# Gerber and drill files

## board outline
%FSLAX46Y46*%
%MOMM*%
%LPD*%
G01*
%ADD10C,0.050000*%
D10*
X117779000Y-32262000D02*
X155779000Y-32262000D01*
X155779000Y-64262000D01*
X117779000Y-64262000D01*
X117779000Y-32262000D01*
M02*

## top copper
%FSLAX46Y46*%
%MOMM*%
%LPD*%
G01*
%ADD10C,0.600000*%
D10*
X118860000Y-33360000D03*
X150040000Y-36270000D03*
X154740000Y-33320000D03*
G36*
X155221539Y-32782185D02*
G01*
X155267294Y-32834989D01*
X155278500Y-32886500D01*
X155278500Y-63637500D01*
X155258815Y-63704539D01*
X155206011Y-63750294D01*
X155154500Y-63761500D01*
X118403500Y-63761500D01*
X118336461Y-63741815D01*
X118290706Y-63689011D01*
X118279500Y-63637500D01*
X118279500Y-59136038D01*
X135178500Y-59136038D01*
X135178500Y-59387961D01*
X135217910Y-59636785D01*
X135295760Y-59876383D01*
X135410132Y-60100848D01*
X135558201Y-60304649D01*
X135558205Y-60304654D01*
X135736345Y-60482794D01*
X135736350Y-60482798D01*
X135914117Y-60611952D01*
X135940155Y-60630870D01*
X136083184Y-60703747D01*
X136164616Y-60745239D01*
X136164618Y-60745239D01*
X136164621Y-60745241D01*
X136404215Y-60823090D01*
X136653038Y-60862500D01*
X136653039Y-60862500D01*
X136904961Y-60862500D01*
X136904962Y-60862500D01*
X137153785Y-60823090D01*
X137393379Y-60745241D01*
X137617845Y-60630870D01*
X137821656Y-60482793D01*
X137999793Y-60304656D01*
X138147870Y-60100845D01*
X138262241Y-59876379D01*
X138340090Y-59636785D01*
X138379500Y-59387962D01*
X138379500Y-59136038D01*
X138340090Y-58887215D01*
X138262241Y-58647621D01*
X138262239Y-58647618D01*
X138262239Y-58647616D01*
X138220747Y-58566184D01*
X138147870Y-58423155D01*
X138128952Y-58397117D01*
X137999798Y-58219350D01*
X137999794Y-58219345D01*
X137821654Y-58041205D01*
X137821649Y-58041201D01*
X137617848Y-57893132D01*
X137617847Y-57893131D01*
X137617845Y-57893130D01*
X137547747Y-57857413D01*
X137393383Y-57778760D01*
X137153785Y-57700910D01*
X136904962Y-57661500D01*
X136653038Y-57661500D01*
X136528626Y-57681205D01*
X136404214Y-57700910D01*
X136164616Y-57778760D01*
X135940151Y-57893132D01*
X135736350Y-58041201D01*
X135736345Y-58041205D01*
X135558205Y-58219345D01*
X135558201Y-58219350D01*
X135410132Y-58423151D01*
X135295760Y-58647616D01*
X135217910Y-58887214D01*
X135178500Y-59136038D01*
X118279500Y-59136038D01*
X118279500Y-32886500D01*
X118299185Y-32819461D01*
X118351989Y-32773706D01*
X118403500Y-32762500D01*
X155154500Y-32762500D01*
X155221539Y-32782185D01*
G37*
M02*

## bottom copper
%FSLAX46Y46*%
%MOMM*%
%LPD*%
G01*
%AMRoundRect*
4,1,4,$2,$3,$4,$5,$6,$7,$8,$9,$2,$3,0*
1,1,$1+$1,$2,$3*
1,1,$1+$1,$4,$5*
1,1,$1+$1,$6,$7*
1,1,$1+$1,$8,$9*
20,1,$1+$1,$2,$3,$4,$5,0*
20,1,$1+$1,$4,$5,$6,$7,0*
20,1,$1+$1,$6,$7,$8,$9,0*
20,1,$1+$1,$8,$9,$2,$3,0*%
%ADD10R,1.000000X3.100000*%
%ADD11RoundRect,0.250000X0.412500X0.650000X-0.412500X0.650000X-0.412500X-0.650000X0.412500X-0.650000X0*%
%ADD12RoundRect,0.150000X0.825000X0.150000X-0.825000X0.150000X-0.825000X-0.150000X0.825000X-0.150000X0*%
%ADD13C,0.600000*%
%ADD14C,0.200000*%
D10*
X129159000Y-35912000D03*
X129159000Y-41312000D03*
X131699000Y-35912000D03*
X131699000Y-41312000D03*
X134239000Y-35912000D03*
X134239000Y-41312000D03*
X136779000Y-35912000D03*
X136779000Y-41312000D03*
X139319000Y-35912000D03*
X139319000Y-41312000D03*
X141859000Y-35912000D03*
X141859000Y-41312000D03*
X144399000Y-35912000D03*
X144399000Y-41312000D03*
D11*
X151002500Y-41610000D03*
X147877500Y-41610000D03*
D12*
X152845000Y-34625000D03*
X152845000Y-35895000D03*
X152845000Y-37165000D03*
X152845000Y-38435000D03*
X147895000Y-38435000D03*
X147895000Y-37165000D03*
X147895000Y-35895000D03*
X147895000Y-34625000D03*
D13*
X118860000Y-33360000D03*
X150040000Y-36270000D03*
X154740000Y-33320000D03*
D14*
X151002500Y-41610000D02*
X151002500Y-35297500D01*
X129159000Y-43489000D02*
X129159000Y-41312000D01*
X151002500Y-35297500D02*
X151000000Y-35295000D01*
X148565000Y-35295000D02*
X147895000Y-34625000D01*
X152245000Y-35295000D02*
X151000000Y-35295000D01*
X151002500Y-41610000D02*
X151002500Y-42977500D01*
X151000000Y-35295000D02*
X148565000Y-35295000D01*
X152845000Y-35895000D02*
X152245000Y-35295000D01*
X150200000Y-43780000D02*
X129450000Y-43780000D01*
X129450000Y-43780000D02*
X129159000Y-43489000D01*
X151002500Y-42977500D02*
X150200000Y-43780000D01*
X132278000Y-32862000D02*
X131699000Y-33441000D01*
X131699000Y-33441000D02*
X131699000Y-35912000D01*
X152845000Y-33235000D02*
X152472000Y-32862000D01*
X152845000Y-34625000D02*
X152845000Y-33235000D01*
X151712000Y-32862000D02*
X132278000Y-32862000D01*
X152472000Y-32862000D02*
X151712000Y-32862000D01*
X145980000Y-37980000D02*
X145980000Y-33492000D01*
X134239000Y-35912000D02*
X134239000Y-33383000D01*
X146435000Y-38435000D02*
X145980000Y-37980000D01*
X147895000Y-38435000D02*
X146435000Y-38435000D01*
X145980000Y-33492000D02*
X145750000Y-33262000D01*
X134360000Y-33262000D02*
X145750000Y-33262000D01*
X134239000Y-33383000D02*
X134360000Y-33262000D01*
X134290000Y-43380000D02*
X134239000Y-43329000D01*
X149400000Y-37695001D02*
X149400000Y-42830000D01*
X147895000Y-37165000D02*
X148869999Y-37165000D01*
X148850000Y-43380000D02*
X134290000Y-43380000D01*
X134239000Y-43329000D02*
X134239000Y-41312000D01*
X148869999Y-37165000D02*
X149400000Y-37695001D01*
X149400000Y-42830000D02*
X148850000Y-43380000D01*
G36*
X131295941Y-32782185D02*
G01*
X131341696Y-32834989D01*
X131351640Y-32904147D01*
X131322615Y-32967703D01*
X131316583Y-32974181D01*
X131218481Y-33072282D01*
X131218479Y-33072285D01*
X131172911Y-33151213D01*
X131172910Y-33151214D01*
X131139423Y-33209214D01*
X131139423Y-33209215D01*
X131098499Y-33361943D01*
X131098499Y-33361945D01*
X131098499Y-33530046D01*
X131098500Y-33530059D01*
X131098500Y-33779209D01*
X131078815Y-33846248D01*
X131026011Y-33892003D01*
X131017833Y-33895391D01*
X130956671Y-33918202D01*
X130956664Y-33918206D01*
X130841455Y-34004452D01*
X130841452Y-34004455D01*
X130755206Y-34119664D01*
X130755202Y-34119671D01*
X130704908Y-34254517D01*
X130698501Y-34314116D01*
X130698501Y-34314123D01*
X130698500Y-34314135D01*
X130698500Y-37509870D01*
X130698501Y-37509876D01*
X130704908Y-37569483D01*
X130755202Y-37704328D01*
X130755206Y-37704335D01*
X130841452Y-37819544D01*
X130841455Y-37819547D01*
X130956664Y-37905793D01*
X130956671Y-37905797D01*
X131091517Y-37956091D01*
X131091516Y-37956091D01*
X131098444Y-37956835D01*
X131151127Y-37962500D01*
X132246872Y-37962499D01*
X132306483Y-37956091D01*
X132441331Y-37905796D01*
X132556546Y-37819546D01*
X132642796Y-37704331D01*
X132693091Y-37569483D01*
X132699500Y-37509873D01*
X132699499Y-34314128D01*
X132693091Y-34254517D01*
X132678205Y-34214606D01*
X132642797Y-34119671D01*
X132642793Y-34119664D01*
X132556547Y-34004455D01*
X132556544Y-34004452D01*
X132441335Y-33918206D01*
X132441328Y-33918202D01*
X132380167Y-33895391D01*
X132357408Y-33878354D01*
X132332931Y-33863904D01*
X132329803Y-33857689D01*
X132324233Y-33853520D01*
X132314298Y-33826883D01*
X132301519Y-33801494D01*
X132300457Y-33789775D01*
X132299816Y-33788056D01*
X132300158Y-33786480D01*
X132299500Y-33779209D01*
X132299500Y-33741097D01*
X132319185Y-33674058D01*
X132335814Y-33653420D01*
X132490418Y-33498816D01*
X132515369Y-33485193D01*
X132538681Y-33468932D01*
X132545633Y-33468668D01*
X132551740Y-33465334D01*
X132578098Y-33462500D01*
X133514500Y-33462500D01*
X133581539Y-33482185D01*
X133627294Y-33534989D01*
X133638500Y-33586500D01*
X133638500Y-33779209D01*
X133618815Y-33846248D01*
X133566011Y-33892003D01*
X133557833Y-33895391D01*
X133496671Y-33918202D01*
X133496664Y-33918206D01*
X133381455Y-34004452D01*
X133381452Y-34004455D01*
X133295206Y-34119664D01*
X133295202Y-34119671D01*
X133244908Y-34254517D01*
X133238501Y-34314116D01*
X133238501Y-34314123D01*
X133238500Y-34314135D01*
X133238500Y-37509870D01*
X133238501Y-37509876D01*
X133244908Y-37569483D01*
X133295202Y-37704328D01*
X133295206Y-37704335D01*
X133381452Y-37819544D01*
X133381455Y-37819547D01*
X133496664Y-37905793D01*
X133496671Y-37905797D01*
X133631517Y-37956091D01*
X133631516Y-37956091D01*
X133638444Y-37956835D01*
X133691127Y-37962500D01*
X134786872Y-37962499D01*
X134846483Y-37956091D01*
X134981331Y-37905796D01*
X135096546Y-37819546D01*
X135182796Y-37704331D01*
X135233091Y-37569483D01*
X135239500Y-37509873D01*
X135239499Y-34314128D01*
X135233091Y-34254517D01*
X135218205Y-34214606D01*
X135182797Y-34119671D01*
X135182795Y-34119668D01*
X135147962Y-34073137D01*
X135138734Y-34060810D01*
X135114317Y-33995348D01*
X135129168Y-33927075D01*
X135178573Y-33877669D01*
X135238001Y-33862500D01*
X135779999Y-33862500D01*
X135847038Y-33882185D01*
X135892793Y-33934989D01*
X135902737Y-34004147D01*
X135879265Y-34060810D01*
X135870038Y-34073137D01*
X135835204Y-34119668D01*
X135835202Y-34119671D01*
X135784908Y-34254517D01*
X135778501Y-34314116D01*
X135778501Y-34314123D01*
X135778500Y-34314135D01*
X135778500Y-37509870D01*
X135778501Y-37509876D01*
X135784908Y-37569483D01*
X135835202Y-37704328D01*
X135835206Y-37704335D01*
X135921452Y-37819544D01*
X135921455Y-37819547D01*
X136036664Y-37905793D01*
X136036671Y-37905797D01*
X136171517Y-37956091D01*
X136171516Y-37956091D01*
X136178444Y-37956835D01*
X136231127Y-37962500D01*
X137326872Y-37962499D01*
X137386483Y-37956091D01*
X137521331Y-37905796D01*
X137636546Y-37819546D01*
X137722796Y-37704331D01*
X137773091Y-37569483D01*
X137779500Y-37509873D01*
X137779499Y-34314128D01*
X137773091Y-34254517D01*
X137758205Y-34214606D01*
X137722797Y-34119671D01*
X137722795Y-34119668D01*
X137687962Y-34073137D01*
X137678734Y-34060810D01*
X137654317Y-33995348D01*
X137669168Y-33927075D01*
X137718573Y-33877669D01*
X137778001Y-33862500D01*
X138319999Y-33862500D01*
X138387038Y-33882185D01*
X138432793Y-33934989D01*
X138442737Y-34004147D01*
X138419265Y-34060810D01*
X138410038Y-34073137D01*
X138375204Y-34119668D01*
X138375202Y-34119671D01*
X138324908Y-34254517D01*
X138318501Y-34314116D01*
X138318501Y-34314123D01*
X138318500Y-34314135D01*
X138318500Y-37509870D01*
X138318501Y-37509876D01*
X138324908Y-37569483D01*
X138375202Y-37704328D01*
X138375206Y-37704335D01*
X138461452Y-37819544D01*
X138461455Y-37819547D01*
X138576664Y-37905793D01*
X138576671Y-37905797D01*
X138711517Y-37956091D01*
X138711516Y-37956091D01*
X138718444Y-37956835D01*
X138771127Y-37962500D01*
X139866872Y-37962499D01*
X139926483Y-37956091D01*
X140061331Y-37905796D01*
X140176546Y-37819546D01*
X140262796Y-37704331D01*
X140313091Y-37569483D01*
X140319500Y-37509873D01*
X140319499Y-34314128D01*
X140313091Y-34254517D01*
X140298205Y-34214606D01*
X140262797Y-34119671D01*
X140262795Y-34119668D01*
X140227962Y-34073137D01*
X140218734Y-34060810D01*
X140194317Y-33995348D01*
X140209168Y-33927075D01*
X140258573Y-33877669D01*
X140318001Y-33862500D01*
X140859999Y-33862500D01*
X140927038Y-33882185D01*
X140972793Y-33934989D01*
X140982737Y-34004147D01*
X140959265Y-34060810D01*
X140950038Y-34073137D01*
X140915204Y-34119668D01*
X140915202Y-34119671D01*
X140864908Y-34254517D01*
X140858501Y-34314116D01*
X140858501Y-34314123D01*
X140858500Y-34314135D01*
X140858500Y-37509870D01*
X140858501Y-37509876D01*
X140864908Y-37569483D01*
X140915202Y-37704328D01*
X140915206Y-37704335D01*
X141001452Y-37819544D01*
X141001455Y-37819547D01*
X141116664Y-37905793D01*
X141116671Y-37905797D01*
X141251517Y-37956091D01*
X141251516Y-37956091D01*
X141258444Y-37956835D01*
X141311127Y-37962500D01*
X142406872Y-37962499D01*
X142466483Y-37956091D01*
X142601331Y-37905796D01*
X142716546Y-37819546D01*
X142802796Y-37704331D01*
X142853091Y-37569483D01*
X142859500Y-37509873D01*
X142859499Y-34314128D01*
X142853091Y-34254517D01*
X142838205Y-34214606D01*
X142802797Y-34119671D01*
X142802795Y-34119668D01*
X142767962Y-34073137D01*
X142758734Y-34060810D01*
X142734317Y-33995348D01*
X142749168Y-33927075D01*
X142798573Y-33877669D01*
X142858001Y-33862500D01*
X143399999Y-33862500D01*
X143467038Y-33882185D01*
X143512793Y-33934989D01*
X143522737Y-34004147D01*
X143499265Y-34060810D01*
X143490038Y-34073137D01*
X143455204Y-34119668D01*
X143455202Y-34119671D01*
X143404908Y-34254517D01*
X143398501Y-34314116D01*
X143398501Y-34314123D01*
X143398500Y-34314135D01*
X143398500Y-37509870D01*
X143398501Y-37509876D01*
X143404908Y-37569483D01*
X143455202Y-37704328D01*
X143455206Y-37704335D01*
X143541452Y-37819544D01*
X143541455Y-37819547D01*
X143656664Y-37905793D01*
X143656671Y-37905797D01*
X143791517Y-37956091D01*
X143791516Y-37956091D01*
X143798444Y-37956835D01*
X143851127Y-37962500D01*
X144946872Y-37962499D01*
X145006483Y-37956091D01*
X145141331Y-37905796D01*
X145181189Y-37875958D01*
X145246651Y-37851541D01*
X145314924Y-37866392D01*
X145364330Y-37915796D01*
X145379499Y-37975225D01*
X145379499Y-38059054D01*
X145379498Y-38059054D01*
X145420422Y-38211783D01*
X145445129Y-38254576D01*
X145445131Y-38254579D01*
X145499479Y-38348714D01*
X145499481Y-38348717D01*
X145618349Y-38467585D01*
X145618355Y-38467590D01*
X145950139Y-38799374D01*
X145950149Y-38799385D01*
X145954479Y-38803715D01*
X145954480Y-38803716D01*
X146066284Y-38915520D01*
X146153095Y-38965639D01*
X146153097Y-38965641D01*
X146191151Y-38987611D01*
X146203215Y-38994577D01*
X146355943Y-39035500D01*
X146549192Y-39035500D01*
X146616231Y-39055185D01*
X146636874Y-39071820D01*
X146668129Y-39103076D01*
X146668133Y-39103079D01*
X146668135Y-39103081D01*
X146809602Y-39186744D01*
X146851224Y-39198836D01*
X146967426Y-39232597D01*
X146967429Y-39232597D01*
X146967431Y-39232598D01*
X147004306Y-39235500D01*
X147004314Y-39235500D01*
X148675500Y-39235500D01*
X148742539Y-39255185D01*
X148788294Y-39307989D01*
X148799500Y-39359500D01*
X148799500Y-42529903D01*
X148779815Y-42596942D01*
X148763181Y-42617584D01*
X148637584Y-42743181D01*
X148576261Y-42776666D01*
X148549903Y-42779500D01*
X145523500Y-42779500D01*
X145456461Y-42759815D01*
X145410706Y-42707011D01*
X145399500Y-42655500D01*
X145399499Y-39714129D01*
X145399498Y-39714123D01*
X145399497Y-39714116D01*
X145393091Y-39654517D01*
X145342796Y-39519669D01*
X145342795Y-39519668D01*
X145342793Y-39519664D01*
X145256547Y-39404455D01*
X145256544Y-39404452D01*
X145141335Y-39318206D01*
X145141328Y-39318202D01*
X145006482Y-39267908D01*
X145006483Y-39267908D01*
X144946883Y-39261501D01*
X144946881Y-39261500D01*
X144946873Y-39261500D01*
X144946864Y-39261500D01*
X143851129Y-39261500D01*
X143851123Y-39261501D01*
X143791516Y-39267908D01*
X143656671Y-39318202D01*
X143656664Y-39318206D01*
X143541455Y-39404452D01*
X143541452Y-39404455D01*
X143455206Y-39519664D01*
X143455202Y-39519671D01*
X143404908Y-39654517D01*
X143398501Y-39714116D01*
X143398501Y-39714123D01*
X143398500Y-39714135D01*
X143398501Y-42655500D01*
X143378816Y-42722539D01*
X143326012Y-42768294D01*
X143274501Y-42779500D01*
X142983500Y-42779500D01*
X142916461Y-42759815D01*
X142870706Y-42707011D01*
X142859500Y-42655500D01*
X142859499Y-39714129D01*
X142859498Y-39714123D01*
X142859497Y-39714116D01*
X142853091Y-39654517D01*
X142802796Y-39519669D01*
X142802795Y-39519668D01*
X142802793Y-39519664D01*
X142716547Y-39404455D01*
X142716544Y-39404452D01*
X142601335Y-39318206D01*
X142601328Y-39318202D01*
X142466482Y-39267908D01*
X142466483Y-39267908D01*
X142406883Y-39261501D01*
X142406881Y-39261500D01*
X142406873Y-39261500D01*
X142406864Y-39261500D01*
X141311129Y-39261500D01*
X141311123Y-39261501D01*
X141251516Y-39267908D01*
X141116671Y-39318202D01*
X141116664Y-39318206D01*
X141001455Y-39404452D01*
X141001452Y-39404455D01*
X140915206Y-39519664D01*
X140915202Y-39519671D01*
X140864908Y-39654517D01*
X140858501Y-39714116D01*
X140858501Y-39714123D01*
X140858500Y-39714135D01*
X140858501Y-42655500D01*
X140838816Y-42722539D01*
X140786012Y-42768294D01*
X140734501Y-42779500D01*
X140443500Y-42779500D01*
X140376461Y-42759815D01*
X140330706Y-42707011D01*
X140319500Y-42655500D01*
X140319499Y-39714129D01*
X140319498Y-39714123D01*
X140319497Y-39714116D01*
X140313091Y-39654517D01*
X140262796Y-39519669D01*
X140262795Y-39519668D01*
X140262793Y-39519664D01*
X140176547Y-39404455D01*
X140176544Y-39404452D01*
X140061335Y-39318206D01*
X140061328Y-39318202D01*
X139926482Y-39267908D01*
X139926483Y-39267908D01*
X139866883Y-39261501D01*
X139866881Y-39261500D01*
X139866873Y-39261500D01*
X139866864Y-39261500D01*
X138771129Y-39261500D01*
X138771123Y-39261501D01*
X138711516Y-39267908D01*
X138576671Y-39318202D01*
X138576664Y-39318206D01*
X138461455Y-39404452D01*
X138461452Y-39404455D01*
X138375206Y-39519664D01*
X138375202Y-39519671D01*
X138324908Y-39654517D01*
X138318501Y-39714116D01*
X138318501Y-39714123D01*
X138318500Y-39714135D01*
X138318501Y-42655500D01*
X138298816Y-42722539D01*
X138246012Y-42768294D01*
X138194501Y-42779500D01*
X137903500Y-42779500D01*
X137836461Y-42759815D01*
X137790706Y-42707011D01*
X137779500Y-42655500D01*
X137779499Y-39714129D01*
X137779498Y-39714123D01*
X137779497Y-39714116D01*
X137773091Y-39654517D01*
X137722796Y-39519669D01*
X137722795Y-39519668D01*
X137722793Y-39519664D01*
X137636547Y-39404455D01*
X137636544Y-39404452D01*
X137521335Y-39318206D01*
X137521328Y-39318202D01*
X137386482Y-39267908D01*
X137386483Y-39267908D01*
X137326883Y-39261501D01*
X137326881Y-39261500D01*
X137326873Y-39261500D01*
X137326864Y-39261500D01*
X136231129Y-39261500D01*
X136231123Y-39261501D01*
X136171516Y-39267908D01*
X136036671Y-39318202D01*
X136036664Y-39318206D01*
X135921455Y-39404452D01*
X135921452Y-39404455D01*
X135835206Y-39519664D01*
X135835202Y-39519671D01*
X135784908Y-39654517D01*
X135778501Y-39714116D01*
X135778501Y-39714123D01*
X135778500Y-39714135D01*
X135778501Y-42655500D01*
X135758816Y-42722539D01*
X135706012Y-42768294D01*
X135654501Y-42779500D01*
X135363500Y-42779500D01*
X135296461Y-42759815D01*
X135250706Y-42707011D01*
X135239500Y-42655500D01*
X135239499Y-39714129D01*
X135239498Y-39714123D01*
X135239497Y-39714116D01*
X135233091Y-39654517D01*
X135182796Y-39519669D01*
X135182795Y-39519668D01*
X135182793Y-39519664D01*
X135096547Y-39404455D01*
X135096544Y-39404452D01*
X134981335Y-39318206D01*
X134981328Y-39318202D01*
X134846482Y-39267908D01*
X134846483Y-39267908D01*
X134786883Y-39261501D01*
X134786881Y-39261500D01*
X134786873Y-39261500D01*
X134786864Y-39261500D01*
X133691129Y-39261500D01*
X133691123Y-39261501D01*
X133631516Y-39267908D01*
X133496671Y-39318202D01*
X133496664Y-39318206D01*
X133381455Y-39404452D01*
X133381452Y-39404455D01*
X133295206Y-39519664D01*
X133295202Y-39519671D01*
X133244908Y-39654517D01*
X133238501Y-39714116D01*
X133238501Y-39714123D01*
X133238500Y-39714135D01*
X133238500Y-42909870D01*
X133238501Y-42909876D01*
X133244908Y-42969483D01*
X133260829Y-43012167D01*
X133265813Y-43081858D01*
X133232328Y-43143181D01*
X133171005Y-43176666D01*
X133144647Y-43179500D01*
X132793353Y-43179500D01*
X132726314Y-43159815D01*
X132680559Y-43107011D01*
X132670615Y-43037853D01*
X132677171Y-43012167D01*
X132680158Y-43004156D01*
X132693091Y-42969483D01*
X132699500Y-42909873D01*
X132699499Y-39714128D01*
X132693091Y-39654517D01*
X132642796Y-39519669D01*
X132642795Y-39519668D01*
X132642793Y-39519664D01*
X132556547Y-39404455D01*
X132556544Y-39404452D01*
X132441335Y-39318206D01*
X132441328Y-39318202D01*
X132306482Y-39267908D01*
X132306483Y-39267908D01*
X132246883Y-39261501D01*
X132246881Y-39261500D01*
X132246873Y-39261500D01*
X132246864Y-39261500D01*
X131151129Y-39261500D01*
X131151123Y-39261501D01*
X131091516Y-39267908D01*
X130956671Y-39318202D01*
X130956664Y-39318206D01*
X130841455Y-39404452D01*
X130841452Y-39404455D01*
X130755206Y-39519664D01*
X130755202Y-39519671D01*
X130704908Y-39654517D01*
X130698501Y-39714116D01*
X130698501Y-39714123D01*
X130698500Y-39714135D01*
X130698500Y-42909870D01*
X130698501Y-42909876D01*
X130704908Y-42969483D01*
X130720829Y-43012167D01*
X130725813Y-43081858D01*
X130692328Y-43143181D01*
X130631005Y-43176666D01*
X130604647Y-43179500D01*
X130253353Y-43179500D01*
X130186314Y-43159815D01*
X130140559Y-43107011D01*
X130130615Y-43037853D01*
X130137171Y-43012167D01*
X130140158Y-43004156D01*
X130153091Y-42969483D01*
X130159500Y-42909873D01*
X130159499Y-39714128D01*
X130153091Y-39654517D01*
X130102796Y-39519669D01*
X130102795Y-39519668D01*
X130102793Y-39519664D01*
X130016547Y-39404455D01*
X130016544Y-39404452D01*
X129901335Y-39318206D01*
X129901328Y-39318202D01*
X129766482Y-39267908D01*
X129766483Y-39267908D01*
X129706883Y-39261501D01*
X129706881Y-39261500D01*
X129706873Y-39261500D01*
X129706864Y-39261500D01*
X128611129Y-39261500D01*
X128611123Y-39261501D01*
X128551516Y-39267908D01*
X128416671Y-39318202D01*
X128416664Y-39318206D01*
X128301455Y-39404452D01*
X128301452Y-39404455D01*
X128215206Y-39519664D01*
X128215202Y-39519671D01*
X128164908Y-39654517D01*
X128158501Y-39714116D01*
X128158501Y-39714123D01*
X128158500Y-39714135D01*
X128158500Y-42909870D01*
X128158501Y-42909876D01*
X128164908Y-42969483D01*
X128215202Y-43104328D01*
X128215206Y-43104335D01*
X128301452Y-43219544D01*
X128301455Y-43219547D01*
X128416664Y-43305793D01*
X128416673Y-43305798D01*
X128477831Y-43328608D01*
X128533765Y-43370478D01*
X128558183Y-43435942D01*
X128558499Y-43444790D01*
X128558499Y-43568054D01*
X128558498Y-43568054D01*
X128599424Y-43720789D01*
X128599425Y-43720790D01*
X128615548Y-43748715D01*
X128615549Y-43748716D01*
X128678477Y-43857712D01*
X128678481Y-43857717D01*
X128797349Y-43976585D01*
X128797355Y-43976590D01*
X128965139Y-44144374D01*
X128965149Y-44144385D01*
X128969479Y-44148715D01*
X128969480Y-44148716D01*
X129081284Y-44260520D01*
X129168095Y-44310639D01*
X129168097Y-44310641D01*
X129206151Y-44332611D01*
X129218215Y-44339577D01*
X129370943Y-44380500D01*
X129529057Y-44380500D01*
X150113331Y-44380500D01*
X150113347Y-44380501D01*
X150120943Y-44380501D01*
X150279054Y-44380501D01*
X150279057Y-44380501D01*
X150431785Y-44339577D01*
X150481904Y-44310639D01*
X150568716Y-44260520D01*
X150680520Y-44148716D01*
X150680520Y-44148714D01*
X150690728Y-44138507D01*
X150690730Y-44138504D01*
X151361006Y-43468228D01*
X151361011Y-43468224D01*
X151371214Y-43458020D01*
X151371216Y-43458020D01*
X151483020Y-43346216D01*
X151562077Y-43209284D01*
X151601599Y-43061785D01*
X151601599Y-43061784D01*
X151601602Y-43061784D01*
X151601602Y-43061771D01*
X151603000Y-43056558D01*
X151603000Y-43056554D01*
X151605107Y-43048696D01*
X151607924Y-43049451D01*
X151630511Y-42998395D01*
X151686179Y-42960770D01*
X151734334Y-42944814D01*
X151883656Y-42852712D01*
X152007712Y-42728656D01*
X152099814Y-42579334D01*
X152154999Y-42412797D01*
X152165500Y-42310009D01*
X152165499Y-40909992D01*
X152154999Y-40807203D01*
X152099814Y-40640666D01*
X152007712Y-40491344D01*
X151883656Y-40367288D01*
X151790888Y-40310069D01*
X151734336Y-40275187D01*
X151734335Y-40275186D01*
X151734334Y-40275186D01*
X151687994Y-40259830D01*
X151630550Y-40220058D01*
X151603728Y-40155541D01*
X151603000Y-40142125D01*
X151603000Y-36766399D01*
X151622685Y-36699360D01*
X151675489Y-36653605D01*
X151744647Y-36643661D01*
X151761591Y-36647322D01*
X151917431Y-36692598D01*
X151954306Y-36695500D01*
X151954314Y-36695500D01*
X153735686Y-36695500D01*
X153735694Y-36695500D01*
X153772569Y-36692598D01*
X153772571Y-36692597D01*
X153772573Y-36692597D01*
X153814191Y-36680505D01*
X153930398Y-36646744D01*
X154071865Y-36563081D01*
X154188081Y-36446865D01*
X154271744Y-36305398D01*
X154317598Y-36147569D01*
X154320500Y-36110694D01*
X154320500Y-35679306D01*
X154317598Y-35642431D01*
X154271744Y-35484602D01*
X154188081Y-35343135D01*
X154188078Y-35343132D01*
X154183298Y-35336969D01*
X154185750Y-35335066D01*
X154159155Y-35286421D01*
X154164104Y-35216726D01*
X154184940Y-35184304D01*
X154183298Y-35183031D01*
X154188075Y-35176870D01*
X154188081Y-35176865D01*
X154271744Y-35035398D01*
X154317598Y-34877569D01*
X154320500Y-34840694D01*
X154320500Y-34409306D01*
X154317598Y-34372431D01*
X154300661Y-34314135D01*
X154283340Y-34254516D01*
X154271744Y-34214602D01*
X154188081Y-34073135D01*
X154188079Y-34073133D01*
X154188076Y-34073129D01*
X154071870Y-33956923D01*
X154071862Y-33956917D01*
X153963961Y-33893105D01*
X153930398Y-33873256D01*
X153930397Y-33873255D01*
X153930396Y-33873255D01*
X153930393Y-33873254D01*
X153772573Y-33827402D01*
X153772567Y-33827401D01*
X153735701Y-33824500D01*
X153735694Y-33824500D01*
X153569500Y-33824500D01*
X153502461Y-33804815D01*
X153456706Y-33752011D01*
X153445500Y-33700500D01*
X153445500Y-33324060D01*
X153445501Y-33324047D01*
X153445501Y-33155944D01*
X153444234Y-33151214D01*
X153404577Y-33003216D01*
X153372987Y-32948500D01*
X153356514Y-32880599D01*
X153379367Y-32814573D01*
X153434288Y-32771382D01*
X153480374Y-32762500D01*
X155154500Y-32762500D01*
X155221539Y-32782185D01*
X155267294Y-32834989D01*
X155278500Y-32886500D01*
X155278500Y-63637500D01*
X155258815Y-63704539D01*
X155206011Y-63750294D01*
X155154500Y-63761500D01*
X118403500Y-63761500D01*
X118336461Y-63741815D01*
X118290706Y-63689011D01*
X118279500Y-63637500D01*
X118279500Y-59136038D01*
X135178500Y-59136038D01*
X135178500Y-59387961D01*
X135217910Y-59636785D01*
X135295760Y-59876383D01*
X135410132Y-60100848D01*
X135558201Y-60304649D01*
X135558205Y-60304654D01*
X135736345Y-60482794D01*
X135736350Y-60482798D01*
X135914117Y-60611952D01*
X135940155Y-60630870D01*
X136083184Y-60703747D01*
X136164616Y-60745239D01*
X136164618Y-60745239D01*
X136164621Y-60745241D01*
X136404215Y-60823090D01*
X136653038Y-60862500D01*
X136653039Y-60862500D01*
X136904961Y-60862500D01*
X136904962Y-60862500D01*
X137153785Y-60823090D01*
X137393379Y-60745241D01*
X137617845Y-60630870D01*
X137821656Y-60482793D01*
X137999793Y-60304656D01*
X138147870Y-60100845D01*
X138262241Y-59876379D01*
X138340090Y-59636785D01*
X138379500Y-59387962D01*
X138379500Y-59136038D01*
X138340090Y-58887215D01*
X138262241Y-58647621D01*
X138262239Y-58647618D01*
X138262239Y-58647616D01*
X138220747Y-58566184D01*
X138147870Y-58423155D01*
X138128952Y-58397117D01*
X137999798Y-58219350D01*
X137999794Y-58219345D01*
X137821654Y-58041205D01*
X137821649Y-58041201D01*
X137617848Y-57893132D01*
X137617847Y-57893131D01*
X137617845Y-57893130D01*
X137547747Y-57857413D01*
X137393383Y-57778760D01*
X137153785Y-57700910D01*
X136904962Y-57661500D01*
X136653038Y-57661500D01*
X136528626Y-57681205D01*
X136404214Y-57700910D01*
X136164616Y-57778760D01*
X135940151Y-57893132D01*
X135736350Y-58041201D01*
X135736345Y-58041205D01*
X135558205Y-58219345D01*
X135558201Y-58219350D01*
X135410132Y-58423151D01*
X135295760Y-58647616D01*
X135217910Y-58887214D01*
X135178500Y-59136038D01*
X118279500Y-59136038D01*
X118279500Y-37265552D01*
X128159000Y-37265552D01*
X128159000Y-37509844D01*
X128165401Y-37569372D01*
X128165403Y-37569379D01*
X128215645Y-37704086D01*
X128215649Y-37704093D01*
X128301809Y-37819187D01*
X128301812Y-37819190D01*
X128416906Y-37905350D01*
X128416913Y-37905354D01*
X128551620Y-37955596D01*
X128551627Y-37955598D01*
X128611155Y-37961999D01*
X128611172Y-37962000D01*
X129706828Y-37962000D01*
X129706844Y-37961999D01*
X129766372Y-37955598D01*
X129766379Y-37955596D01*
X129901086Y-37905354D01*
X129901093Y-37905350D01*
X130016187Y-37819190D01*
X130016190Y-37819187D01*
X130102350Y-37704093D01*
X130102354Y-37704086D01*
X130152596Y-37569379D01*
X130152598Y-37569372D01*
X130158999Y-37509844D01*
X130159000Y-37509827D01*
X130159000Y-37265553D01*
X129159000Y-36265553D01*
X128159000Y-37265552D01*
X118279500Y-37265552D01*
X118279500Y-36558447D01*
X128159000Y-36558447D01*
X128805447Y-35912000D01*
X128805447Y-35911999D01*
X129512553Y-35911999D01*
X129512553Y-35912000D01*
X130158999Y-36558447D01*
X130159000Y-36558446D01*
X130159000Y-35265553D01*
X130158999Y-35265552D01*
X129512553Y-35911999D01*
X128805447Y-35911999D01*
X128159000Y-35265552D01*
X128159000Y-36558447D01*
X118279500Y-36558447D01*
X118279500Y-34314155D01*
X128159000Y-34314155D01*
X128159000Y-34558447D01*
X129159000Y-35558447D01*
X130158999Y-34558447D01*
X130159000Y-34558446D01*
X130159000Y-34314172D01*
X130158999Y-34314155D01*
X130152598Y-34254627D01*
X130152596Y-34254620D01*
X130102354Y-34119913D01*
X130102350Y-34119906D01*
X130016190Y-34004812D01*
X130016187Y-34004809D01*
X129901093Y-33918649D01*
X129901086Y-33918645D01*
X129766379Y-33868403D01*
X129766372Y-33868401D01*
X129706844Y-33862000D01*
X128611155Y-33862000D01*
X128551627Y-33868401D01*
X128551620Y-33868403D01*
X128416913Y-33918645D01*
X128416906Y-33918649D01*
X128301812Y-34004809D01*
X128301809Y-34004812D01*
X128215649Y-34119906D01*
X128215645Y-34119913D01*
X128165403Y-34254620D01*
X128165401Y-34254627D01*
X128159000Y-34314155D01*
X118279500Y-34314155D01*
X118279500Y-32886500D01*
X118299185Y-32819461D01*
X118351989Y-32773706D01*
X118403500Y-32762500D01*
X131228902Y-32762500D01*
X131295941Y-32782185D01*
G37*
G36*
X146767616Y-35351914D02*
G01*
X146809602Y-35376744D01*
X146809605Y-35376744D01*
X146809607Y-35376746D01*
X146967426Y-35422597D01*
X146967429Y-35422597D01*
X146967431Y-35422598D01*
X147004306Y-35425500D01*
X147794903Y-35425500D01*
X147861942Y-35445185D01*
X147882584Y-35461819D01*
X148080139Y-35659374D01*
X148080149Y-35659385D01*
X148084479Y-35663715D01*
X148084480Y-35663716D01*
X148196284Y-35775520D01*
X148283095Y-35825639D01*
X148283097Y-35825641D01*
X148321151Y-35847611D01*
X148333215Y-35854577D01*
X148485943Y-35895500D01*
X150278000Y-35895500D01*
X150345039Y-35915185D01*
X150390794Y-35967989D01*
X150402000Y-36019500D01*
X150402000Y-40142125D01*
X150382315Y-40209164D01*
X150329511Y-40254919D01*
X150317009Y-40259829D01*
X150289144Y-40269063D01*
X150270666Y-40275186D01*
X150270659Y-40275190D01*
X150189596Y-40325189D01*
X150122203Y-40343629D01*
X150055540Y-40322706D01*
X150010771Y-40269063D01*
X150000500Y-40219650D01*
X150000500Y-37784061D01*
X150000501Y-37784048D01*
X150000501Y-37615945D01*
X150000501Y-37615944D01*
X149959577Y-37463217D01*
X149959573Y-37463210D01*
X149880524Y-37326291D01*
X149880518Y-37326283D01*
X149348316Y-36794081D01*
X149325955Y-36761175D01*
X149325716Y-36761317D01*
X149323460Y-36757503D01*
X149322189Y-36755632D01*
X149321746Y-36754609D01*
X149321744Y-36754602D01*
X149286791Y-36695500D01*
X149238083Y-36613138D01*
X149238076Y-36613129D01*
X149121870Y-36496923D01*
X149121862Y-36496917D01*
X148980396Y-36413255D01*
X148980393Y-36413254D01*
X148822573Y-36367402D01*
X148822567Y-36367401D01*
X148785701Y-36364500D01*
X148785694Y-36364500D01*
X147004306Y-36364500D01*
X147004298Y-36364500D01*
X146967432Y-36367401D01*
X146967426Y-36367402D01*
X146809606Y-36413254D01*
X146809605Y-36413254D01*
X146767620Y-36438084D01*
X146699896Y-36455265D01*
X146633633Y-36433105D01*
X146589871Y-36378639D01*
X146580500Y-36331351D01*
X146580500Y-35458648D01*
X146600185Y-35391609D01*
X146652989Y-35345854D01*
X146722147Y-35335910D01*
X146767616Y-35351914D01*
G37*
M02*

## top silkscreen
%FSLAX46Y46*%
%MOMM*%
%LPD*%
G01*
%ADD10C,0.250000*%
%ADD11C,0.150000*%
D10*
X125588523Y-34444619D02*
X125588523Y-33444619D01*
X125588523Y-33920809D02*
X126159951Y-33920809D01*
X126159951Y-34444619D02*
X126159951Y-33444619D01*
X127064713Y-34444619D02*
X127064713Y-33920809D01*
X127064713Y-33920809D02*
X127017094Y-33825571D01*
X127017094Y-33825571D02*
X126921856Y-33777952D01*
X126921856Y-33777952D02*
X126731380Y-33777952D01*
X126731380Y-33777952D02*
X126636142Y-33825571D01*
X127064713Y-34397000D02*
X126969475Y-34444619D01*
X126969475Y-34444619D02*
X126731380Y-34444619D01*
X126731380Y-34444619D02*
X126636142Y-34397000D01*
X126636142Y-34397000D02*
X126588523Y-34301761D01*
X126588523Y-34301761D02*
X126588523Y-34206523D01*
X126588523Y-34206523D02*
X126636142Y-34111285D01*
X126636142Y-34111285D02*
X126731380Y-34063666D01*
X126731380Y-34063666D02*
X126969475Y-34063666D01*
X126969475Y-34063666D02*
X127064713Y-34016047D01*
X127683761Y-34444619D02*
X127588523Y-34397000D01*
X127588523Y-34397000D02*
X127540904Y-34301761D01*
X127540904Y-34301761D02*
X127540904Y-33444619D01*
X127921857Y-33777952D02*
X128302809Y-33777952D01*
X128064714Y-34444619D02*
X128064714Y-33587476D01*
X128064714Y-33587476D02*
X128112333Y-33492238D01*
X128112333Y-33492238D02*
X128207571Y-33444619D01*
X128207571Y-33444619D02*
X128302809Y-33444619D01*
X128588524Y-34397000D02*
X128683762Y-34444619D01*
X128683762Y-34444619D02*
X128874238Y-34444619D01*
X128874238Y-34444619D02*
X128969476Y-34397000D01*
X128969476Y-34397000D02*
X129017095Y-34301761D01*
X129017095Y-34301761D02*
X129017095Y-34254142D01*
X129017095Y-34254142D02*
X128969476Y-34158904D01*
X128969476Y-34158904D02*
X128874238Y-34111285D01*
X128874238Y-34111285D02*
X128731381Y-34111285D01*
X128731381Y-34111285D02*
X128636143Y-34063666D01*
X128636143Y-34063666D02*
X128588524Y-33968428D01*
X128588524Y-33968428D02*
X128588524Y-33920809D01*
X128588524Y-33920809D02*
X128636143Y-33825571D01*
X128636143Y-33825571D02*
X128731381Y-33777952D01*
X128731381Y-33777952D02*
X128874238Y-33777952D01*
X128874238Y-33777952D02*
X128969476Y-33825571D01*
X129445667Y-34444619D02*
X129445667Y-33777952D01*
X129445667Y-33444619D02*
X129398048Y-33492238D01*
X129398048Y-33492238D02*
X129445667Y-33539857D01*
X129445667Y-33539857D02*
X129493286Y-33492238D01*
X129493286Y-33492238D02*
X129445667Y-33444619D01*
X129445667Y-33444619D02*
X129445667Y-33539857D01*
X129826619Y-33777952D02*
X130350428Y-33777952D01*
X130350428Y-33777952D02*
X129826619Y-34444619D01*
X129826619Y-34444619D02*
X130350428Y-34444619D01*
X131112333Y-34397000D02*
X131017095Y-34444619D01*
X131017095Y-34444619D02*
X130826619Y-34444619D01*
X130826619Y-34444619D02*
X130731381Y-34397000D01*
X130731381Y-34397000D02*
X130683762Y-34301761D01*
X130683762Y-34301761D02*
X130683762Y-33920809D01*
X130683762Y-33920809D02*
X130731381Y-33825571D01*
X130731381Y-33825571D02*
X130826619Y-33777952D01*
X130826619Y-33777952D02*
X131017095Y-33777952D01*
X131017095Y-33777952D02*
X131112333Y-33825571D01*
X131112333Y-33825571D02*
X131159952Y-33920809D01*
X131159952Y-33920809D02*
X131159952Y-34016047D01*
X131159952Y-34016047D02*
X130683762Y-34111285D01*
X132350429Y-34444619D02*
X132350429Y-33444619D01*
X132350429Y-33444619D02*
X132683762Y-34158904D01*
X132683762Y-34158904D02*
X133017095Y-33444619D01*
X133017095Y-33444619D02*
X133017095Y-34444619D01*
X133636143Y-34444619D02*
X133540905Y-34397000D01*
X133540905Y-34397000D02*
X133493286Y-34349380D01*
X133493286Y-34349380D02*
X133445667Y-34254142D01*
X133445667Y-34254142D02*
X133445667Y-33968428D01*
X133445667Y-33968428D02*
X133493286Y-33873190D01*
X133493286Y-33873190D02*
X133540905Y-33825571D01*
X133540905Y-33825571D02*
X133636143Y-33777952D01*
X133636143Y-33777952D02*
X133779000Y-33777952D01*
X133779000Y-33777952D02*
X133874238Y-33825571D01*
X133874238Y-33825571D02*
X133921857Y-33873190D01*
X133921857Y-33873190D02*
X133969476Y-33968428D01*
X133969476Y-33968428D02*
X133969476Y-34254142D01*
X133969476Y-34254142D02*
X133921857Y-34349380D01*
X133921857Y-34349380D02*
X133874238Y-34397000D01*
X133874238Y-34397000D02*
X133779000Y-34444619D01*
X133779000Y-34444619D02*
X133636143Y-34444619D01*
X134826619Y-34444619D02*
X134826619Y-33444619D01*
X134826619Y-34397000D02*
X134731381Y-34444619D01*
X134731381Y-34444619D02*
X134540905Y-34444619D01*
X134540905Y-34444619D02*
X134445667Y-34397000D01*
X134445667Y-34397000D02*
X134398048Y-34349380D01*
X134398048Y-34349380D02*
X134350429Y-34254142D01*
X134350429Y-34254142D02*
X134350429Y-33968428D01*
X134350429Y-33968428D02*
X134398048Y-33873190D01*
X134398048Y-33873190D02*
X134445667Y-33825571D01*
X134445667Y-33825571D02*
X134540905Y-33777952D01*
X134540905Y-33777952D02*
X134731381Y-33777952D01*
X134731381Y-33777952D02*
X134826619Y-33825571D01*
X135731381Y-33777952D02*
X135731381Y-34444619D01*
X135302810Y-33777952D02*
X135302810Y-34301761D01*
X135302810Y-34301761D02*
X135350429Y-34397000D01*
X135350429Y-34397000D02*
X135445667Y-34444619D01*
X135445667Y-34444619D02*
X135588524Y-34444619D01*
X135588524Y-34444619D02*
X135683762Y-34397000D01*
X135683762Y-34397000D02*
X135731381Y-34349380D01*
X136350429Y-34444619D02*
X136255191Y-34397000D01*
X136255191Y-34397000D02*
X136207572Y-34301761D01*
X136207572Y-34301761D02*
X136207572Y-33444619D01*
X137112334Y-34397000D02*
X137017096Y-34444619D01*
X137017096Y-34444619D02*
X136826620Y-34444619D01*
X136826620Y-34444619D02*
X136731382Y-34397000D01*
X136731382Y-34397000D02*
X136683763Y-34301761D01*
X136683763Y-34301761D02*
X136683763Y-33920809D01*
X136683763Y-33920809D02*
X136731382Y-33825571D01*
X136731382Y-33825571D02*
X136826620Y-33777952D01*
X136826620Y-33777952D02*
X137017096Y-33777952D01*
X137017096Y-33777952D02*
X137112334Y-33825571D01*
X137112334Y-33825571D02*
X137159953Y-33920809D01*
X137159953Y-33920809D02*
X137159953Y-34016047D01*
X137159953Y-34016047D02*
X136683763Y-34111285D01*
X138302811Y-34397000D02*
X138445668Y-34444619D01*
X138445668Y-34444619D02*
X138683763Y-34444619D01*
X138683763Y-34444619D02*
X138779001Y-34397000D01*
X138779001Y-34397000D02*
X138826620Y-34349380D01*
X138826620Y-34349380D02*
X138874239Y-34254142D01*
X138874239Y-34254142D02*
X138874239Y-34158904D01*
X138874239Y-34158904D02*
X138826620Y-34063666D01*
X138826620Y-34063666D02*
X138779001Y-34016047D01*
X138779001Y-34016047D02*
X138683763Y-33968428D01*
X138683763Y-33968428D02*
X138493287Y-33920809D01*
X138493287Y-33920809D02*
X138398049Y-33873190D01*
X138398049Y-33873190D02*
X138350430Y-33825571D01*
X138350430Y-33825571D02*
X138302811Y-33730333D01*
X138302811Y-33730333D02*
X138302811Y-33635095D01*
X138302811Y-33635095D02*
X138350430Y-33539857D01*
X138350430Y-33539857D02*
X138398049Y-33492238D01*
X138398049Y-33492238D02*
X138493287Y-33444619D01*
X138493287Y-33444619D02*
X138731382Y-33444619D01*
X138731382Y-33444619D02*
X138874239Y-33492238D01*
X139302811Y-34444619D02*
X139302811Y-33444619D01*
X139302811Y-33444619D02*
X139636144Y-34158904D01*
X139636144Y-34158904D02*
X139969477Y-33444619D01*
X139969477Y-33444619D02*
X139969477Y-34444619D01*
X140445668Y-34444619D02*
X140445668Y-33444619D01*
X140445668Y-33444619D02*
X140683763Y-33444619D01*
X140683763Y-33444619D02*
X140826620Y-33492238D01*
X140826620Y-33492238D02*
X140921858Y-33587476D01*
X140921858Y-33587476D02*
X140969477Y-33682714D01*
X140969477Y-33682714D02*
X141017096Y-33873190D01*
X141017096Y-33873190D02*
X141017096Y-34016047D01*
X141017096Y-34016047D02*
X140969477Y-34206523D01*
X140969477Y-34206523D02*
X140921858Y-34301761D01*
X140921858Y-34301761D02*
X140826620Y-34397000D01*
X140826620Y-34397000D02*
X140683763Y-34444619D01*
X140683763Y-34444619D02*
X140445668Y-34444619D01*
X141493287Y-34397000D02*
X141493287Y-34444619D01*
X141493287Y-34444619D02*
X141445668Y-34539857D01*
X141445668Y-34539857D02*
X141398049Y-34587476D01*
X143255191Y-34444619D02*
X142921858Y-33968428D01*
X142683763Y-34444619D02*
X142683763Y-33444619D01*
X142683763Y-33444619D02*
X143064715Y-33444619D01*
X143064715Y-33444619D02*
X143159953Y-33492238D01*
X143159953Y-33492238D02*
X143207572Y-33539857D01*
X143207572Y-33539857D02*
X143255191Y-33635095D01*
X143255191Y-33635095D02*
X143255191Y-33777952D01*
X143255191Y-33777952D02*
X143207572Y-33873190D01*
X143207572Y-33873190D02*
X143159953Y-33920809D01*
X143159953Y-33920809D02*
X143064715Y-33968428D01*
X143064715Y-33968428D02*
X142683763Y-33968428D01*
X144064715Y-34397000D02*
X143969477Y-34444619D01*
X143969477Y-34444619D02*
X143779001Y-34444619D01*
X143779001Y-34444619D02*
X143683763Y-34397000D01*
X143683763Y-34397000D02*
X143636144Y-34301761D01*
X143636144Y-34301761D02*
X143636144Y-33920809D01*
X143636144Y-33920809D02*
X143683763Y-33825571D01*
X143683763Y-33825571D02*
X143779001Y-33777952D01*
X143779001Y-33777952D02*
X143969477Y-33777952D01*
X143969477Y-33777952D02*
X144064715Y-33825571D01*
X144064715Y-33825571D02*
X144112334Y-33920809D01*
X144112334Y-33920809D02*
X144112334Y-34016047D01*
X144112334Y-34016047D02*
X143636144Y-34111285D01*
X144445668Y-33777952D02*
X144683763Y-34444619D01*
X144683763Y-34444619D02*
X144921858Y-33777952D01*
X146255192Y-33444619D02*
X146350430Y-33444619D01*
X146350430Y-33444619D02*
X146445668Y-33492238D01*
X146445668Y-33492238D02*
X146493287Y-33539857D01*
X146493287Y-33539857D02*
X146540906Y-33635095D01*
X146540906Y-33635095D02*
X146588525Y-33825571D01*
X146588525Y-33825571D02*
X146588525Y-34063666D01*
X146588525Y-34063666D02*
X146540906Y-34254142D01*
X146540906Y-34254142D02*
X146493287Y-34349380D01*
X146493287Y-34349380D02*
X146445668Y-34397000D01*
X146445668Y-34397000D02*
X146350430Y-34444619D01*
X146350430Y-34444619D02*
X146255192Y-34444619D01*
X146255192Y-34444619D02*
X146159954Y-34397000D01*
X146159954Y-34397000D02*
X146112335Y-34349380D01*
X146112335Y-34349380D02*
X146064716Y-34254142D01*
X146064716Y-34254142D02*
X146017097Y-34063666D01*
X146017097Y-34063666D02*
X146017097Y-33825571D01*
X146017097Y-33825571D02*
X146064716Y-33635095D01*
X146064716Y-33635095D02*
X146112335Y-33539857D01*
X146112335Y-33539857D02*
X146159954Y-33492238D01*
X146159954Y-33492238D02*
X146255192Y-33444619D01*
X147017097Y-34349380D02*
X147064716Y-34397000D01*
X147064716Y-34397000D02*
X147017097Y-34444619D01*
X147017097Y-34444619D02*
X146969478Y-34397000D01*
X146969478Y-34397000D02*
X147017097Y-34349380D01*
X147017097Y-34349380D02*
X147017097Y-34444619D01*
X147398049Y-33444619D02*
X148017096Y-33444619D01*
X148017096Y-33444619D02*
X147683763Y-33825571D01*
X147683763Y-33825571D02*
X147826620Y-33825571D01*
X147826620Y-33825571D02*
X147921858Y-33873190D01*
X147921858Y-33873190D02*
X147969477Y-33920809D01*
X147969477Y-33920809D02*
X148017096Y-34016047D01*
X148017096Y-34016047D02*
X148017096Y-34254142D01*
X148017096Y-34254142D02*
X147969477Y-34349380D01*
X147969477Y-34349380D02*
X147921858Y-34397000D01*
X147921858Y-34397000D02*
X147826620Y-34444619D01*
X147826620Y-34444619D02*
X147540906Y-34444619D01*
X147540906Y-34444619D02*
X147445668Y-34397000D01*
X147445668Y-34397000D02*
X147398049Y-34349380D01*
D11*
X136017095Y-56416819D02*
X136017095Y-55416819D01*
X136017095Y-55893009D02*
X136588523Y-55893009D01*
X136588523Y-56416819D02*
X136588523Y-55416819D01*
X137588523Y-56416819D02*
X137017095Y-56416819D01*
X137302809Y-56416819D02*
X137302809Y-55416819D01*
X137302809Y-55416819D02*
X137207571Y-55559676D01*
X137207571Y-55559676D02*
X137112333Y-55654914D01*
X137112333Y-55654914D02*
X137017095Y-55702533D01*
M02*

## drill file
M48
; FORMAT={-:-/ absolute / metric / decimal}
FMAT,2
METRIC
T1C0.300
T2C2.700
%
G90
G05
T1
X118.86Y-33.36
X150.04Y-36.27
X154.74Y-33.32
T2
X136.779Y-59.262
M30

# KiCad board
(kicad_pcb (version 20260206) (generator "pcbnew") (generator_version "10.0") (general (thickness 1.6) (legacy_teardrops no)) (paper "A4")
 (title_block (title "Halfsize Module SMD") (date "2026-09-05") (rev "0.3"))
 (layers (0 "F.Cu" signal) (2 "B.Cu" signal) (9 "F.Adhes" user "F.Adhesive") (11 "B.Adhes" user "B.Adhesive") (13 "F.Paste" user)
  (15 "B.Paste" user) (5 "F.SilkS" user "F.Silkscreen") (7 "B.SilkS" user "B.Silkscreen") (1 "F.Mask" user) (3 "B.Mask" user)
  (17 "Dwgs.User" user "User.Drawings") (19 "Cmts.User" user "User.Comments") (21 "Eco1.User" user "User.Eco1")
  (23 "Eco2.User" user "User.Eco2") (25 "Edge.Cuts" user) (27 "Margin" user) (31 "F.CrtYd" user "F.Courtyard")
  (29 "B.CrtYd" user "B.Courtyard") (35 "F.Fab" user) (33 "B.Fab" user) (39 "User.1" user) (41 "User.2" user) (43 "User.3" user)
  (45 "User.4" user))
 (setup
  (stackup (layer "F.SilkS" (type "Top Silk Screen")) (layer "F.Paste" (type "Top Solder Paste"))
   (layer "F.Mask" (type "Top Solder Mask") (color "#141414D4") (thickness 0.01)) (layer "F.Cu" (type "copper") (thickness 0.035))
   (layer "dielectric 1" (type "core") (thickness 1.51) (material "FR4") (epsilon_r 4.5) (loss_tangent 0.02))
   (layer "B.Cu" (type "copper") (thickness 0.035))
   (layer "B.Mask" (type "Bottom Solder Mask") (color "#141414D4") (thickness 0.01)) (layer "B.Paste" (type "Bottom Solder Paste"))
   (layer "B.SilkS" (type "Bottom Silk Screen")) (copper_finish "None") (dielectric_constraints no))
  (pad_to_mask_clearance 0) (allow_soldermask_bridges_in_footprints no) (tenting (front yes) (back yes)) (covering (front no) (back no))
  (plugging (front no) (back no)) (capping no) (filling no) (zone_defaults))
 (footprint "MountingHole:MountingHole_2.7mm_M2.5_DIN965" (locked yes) (layer "F.Cu") (at 136.779 59.262)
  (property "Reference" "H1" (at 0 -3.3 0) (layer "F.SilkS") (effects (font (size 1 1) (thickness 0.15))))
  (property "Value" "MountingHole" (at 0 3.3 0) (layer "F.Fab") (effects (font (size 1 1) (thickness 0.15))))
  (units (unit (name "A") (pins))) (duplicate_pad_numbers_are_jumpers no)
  (pad "" np_thru_hole circle (at 0 0) (size 2.7 2.7) (drill 2.7) (layers "*.Cu" "*.Mask")))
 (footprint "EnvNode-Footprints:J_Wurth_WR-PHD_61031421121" (layer "B.Cu") (at 136.779 38.612 -90)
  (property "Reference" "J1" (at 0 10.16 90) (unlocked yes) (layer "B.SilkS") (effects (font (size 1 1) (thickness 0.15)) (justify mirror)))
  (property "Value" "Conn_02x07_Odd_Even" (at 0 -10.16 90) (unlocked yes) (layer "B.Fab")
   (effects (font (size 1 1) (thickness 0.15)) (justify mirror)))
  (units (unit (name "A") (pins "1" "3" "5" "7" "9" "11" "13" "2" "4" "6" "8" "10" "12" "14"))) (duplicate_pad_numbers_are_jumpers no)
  (pad "1" smd rect (at -2.7 7.62) (size 1 3.1) (layers "B.Cu" "B.Mask" "B.Paste") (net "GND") (thermal_bridge_angle 45))
  (pad "2" smd rect (at 2.7 7.62) (size 1 3.1) (layers "B.Cu" "B.Mask" "B.Paste") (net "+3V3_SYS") (thermal_bridge_angle 45))
  (pad "3" smd rect (at -2.7 5.08) (size 1 3.1) (layers "B.Cu" "B.Mask" "B.Paste") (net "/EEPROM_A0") (thermal_bridge_angle 45))
  (pad "4" smd rect (at 2.7 5.08) (size 1 3.1) (layers "B.Cu" "B.Mask" "B.Paste") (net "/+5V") (thermal_bridge_angle 45))
  (pad "5" smd rect (at -2.7 2.54) (size 1 3.1) (layers "B.Cu" "B.Mask" "B.Paste") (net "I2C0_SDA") (thermal_bridge_angle 45))
  (pad "6" smd rect (at 2.7 2.54) (size 1 3.1) (layers "B.Cu" "B.Mask" "B.Paste") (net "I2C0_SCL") (thermal_bridge_angle 45))
  (pad "7" smd rect (at -2.7 0) (size 1 3.1) (layers "B.Cu" "B.Mask" "B.Paste") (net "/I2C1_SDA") (thermal_bridge_angle 45))
  (pad "8" smd rect (at 2.7 0) (size 1 3.1) (layers "B.Cu" "B.Mask" "B.Paste") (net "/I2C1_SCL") (thermal_bridge_angle 45))
  (pad "9" smd rect (at -2.7 -2.54) (size 1 3.1) (layers "B.Cu" "B.Mask" "B.Paste") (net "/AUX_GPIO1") (thermal_bridge_angle 45))
  (pad "10" smd rect (at 2.7 -2.54) (size 1 3.1) (layers "B.Cu" "B.Mask" "B.Paste") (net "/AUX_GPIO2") (thermal_bridge_angle 45))
  (pad "11" smd rect (at -2.7 -5.08) (size 1 3.1) (layers "B.Cu" "B.Mask" "B.Paste") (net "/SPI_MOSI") (thermal_bridge_angle 45))
  (pad "12" smd rect (at 2.7 -5.08) (size 1 3.1) (layers "B.Cu" "B.Mask" "B.Paste") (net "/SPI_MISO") (thermal_bridge_angle 45))
  (pad "13" smd rect (at -2.7 -7.62) (size 1 3.1) (layers "B.Cu" "B.Mask" "B.Paste") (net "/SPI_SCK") (thermal_bridge_angle 45))
  (pad "14" smd rect (at 2.7 -7.62) (size 1 3.1) (layers "B.Cu" "B.Mask" "B.Paste") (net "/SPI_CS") (thermal_bridge_angle 45)))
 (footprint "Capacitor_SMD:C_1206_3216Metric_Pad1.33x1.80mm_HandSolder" (layer "B.Cu") (at 149.44 41.61 180)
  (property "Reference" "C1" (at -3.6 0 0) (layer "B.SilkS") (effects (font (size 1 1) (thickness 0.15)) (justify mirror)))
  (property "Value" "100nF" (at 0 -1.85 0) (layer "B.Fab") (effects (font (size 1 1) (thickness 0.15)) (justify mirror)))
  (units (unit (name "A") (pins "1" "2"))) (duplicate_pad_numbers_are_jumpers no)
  (pad "1" smd roundrect (at -1.5625 0 180) (size 1.325 1.8) (layers "B.Cu" "B.Mask" "B.Paste") (roundrect_rratio 0.188679) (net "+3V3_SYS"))
  (pad "2" smd roundrect (at 1.5625 0 180) (size 1.325 1.8) (layers "B.Cu" "B.Mask" "B.Paste") (roundrect_rratio 0.188679) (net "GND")
   (zone_connect 2)))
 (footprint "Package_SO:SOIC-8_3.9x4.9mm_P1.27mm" (layer "B.Cu") (at 150.37 36.53 180)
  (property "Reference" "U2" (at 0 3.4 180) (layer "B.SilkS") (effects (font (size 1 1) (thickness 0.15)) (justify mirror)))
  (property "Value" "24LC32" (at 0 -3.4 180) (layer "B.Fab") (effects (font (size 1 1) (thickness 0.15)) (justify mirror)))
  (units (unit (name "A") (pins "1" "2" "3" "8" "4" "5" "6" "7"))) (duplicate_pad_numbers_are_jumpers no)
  (pad "1" smd roundrect (at -2.475 1.905 180) (size 1.95 0.6) (layers "B.Cu" "B.Mask" "B.Paste") (roundrect_rratio 0.25) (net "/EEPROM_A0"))
  (pad "2" smd roundrect (at -2.475 0.635 180) (size 1.95 0.6) (layers "B.Cu" "B.Mask" "B.Paste") (roundrect_rratio 0.25) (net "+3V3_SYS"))
  (pad "3" smd roundrect (at -2.475 -0.635 180) (size 1.95 0.6) (layers "B.Cu" "B.Mask" "B.Paste") (roundrect_rratio 0.25) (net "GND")
   (zone_connect 2))
  (pad "4" smd roundrect (at -2.475 -1.905 180) (size 1.95 0.6) (layers "B.Cu" "B.Mask" "B.Paste") (roundrect_rratio 0.25) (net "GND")
   (zone_connect 2))
  (pad "5" smd roundrect (at 2.475 -1.905 180) (size 1.95 0.6) (layers "B.Cu" "B.Mask" "B.Paste") (roundrect_rratio 0.25) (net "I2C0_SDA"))
  (pad "6" smd roundrect (at 2.475 -0.635 180) (size 1.95 0.6) (layers "B.Cu" "B.Mask" "B.Paste") (roundrect_rratio 0.25) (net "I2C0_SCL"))
  (pad "7" smd roundrect (at 2.475 0.635 180) (size 1.95 0.6) (layers "B.Cu" "B.Mask" "B.Paste") (roundrect_rratio 0.25) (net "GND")
   (zone_connect 2))
  (pad "8" smd roundrect (at 2.475 1.905 180) (size 1.95 0.6) (layers "B.Cu" "B.Mask" "B.Paste") (roundrect_rratio 0.25) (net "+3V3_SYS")))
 (gr_rect (start 117.779 32.262) (end 155.779 64.262) (stroke (width 0.05) (type solid)) (fill no) (layer "Edge.Cuts"))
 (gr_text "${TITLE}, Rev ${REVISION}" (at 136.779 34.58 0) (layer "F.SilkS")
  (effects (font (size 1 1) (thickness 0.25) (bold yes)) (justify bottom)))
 (via (at 118.86 33.36) (size 0.6) (drill 0.3) (layers "F.Cu" "B.Cu") (free yes) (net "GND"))
 (via (at 150.04 36.27) (size 0.6) (drill 0.3) (layers "F.Cu" "B.Cu") (free yes) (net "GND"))
 (via (at 154.74 33.32) (size 0.6) (drill 0.3) (layers "F.Cu" "B.Cu") (free yes) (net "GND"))
 (segment (start 151.0025 41.61) (end 151.0025 35.2975) (width 0.2) (layer "B.Cu") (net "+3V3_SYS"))
 (segment (start 129.159 43.489) (end 129.159 41.312) (width 0.2) (layer "B.Cu") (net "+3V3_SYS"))
 (segment (start 151.0025 35.2975) (end 151 35.295) (width 0.2) (layer "B.Cu") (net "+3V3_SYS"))
 (segment (start 148.565 35.295) (end 147.895 34.625) (width 0.2) (layer "B.Cu") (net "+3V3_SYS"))
 (segment (start 152.245 35.295) (end 151 35.295) (width 0.2) (layer "B.Cu") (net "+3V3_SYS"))
 (segment (start 151.0025 41.61) (end 151.0025 42.9775) (width 0.2) (layer "B.Cu") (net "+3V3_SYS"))
 (segment (start 151 35.295) (end 148.565 35.295) (width 0.2) (layer "B.Cu") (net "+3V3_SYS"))
 (segment (start 152.845 35.895) (end 152.245 35.295) (width 0.2) (layer "B.Cu") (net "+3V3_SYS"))
 (segment (start 150.2 43.78) (end 129.45 43.78) (width 0.2) (layer "B.Cu") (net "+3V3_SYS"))
 (segment (start 129.45 43.78) (end 129.159 43.489) (width 0.2) (layer "B.Cu") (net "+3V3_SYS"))
 (segment (start 151.0025 42.9775) (end 150.2 43.78) (width 0.2) (layer "B.Cu") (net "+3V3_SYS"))
 (segment (start 132.278 32.862) (end 131.699 33.441) (width 0.2) (layer "B.Cu") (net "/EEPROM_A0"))
 (segment (start 131.699 33.441) (end 131.699 35.912) (width 0.2) (layer "B.Cu") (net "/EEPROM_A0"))
 (segment (start 152.845 33.235) (end 152.472 32.862) (width 0.2) (layer "B.Cu") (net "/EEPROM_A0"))
 (segment (start 152.845 34.625) (end 152.845 33.235) (width 0.2) (layer "B.Cu") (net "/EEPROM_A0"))
 (segment (start 151.712 32.862) (end 132.278 32.862) (width 0.2) (layer "B.Cu") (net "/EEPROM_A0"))
 (segment (start 152.472 32.862) (end 151.712 32.862) (width 0.2) (layer "B.Cu") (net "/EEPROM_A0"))
 (segment (start 145.98 37.98) (end 145.98 33.492) (width 0.2) (layer "B.Cu") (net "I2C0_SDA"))
 (segment (start 134.239 35.912) (end 134.239 33.383) (width 0.2) (layer "B.Cu") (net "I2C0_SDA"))
 (segment (start 146.435 38.435) (end 145.98 37.98) (width 0.2) (layer "B.Cu") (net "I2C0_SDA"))
 (segment (start 147.895 38.435) (end 146.435 38.435) (width 0.2) (layer "B.Cu") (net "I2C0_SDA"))
 (segment (start 145.98 33.492) (end 145.75 33.262) (width 0.2) (layer "B.Cu") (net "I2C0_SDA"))
 (segment (start 134.36 33.262) (end 145.75 33.262) (width 0.2) (layer "B.Cu") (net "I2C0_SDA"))
 (segment (start 134.239 33.383) (end 134.36 33.262) (width 0.2) (layer "B.Cu") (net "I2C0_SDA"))
 (segment (start 134.29 43.38) (end 134.239 43.329) (width 0.2) (layer "B.Cu") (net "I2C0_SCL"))
 (segment (start 149.4 37.695001) (end 149.4 42.83) (width 0.2) (layer "B.Cu") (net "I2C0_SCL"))
 (segment (start 147.895 37.165) (end 148.869999 37.165) (width 0.2) (layer "B.Cu") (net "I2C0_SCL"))
 (segment (start 148.85 43.38) (end 134.29 43.38) (width 0.2) (layer "B.Cu") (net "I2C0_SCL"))
 (segment (start 134.239 43.329) (end 134.239 41.312) (width 0.2) (layer "B.Cu") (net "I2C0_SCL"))
 (segment (start 148.869999 37.165) (end 149.4 37.695001) (width 0.2) (layer "B.Cu") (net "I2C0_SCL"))
 (segment (start 149.4 42.83) (end 148.85 43.38) (width 0.2) (layer "B.Cu") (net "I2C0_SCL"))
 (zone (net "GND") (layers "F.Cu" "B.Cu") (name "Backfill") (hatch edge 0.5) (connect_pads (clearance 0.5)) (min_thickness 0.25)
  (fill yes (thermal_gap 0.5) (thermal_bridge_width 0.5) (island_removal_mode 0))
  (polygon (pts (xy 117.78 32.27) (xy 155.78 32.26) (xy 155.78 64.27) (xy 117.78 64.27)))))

